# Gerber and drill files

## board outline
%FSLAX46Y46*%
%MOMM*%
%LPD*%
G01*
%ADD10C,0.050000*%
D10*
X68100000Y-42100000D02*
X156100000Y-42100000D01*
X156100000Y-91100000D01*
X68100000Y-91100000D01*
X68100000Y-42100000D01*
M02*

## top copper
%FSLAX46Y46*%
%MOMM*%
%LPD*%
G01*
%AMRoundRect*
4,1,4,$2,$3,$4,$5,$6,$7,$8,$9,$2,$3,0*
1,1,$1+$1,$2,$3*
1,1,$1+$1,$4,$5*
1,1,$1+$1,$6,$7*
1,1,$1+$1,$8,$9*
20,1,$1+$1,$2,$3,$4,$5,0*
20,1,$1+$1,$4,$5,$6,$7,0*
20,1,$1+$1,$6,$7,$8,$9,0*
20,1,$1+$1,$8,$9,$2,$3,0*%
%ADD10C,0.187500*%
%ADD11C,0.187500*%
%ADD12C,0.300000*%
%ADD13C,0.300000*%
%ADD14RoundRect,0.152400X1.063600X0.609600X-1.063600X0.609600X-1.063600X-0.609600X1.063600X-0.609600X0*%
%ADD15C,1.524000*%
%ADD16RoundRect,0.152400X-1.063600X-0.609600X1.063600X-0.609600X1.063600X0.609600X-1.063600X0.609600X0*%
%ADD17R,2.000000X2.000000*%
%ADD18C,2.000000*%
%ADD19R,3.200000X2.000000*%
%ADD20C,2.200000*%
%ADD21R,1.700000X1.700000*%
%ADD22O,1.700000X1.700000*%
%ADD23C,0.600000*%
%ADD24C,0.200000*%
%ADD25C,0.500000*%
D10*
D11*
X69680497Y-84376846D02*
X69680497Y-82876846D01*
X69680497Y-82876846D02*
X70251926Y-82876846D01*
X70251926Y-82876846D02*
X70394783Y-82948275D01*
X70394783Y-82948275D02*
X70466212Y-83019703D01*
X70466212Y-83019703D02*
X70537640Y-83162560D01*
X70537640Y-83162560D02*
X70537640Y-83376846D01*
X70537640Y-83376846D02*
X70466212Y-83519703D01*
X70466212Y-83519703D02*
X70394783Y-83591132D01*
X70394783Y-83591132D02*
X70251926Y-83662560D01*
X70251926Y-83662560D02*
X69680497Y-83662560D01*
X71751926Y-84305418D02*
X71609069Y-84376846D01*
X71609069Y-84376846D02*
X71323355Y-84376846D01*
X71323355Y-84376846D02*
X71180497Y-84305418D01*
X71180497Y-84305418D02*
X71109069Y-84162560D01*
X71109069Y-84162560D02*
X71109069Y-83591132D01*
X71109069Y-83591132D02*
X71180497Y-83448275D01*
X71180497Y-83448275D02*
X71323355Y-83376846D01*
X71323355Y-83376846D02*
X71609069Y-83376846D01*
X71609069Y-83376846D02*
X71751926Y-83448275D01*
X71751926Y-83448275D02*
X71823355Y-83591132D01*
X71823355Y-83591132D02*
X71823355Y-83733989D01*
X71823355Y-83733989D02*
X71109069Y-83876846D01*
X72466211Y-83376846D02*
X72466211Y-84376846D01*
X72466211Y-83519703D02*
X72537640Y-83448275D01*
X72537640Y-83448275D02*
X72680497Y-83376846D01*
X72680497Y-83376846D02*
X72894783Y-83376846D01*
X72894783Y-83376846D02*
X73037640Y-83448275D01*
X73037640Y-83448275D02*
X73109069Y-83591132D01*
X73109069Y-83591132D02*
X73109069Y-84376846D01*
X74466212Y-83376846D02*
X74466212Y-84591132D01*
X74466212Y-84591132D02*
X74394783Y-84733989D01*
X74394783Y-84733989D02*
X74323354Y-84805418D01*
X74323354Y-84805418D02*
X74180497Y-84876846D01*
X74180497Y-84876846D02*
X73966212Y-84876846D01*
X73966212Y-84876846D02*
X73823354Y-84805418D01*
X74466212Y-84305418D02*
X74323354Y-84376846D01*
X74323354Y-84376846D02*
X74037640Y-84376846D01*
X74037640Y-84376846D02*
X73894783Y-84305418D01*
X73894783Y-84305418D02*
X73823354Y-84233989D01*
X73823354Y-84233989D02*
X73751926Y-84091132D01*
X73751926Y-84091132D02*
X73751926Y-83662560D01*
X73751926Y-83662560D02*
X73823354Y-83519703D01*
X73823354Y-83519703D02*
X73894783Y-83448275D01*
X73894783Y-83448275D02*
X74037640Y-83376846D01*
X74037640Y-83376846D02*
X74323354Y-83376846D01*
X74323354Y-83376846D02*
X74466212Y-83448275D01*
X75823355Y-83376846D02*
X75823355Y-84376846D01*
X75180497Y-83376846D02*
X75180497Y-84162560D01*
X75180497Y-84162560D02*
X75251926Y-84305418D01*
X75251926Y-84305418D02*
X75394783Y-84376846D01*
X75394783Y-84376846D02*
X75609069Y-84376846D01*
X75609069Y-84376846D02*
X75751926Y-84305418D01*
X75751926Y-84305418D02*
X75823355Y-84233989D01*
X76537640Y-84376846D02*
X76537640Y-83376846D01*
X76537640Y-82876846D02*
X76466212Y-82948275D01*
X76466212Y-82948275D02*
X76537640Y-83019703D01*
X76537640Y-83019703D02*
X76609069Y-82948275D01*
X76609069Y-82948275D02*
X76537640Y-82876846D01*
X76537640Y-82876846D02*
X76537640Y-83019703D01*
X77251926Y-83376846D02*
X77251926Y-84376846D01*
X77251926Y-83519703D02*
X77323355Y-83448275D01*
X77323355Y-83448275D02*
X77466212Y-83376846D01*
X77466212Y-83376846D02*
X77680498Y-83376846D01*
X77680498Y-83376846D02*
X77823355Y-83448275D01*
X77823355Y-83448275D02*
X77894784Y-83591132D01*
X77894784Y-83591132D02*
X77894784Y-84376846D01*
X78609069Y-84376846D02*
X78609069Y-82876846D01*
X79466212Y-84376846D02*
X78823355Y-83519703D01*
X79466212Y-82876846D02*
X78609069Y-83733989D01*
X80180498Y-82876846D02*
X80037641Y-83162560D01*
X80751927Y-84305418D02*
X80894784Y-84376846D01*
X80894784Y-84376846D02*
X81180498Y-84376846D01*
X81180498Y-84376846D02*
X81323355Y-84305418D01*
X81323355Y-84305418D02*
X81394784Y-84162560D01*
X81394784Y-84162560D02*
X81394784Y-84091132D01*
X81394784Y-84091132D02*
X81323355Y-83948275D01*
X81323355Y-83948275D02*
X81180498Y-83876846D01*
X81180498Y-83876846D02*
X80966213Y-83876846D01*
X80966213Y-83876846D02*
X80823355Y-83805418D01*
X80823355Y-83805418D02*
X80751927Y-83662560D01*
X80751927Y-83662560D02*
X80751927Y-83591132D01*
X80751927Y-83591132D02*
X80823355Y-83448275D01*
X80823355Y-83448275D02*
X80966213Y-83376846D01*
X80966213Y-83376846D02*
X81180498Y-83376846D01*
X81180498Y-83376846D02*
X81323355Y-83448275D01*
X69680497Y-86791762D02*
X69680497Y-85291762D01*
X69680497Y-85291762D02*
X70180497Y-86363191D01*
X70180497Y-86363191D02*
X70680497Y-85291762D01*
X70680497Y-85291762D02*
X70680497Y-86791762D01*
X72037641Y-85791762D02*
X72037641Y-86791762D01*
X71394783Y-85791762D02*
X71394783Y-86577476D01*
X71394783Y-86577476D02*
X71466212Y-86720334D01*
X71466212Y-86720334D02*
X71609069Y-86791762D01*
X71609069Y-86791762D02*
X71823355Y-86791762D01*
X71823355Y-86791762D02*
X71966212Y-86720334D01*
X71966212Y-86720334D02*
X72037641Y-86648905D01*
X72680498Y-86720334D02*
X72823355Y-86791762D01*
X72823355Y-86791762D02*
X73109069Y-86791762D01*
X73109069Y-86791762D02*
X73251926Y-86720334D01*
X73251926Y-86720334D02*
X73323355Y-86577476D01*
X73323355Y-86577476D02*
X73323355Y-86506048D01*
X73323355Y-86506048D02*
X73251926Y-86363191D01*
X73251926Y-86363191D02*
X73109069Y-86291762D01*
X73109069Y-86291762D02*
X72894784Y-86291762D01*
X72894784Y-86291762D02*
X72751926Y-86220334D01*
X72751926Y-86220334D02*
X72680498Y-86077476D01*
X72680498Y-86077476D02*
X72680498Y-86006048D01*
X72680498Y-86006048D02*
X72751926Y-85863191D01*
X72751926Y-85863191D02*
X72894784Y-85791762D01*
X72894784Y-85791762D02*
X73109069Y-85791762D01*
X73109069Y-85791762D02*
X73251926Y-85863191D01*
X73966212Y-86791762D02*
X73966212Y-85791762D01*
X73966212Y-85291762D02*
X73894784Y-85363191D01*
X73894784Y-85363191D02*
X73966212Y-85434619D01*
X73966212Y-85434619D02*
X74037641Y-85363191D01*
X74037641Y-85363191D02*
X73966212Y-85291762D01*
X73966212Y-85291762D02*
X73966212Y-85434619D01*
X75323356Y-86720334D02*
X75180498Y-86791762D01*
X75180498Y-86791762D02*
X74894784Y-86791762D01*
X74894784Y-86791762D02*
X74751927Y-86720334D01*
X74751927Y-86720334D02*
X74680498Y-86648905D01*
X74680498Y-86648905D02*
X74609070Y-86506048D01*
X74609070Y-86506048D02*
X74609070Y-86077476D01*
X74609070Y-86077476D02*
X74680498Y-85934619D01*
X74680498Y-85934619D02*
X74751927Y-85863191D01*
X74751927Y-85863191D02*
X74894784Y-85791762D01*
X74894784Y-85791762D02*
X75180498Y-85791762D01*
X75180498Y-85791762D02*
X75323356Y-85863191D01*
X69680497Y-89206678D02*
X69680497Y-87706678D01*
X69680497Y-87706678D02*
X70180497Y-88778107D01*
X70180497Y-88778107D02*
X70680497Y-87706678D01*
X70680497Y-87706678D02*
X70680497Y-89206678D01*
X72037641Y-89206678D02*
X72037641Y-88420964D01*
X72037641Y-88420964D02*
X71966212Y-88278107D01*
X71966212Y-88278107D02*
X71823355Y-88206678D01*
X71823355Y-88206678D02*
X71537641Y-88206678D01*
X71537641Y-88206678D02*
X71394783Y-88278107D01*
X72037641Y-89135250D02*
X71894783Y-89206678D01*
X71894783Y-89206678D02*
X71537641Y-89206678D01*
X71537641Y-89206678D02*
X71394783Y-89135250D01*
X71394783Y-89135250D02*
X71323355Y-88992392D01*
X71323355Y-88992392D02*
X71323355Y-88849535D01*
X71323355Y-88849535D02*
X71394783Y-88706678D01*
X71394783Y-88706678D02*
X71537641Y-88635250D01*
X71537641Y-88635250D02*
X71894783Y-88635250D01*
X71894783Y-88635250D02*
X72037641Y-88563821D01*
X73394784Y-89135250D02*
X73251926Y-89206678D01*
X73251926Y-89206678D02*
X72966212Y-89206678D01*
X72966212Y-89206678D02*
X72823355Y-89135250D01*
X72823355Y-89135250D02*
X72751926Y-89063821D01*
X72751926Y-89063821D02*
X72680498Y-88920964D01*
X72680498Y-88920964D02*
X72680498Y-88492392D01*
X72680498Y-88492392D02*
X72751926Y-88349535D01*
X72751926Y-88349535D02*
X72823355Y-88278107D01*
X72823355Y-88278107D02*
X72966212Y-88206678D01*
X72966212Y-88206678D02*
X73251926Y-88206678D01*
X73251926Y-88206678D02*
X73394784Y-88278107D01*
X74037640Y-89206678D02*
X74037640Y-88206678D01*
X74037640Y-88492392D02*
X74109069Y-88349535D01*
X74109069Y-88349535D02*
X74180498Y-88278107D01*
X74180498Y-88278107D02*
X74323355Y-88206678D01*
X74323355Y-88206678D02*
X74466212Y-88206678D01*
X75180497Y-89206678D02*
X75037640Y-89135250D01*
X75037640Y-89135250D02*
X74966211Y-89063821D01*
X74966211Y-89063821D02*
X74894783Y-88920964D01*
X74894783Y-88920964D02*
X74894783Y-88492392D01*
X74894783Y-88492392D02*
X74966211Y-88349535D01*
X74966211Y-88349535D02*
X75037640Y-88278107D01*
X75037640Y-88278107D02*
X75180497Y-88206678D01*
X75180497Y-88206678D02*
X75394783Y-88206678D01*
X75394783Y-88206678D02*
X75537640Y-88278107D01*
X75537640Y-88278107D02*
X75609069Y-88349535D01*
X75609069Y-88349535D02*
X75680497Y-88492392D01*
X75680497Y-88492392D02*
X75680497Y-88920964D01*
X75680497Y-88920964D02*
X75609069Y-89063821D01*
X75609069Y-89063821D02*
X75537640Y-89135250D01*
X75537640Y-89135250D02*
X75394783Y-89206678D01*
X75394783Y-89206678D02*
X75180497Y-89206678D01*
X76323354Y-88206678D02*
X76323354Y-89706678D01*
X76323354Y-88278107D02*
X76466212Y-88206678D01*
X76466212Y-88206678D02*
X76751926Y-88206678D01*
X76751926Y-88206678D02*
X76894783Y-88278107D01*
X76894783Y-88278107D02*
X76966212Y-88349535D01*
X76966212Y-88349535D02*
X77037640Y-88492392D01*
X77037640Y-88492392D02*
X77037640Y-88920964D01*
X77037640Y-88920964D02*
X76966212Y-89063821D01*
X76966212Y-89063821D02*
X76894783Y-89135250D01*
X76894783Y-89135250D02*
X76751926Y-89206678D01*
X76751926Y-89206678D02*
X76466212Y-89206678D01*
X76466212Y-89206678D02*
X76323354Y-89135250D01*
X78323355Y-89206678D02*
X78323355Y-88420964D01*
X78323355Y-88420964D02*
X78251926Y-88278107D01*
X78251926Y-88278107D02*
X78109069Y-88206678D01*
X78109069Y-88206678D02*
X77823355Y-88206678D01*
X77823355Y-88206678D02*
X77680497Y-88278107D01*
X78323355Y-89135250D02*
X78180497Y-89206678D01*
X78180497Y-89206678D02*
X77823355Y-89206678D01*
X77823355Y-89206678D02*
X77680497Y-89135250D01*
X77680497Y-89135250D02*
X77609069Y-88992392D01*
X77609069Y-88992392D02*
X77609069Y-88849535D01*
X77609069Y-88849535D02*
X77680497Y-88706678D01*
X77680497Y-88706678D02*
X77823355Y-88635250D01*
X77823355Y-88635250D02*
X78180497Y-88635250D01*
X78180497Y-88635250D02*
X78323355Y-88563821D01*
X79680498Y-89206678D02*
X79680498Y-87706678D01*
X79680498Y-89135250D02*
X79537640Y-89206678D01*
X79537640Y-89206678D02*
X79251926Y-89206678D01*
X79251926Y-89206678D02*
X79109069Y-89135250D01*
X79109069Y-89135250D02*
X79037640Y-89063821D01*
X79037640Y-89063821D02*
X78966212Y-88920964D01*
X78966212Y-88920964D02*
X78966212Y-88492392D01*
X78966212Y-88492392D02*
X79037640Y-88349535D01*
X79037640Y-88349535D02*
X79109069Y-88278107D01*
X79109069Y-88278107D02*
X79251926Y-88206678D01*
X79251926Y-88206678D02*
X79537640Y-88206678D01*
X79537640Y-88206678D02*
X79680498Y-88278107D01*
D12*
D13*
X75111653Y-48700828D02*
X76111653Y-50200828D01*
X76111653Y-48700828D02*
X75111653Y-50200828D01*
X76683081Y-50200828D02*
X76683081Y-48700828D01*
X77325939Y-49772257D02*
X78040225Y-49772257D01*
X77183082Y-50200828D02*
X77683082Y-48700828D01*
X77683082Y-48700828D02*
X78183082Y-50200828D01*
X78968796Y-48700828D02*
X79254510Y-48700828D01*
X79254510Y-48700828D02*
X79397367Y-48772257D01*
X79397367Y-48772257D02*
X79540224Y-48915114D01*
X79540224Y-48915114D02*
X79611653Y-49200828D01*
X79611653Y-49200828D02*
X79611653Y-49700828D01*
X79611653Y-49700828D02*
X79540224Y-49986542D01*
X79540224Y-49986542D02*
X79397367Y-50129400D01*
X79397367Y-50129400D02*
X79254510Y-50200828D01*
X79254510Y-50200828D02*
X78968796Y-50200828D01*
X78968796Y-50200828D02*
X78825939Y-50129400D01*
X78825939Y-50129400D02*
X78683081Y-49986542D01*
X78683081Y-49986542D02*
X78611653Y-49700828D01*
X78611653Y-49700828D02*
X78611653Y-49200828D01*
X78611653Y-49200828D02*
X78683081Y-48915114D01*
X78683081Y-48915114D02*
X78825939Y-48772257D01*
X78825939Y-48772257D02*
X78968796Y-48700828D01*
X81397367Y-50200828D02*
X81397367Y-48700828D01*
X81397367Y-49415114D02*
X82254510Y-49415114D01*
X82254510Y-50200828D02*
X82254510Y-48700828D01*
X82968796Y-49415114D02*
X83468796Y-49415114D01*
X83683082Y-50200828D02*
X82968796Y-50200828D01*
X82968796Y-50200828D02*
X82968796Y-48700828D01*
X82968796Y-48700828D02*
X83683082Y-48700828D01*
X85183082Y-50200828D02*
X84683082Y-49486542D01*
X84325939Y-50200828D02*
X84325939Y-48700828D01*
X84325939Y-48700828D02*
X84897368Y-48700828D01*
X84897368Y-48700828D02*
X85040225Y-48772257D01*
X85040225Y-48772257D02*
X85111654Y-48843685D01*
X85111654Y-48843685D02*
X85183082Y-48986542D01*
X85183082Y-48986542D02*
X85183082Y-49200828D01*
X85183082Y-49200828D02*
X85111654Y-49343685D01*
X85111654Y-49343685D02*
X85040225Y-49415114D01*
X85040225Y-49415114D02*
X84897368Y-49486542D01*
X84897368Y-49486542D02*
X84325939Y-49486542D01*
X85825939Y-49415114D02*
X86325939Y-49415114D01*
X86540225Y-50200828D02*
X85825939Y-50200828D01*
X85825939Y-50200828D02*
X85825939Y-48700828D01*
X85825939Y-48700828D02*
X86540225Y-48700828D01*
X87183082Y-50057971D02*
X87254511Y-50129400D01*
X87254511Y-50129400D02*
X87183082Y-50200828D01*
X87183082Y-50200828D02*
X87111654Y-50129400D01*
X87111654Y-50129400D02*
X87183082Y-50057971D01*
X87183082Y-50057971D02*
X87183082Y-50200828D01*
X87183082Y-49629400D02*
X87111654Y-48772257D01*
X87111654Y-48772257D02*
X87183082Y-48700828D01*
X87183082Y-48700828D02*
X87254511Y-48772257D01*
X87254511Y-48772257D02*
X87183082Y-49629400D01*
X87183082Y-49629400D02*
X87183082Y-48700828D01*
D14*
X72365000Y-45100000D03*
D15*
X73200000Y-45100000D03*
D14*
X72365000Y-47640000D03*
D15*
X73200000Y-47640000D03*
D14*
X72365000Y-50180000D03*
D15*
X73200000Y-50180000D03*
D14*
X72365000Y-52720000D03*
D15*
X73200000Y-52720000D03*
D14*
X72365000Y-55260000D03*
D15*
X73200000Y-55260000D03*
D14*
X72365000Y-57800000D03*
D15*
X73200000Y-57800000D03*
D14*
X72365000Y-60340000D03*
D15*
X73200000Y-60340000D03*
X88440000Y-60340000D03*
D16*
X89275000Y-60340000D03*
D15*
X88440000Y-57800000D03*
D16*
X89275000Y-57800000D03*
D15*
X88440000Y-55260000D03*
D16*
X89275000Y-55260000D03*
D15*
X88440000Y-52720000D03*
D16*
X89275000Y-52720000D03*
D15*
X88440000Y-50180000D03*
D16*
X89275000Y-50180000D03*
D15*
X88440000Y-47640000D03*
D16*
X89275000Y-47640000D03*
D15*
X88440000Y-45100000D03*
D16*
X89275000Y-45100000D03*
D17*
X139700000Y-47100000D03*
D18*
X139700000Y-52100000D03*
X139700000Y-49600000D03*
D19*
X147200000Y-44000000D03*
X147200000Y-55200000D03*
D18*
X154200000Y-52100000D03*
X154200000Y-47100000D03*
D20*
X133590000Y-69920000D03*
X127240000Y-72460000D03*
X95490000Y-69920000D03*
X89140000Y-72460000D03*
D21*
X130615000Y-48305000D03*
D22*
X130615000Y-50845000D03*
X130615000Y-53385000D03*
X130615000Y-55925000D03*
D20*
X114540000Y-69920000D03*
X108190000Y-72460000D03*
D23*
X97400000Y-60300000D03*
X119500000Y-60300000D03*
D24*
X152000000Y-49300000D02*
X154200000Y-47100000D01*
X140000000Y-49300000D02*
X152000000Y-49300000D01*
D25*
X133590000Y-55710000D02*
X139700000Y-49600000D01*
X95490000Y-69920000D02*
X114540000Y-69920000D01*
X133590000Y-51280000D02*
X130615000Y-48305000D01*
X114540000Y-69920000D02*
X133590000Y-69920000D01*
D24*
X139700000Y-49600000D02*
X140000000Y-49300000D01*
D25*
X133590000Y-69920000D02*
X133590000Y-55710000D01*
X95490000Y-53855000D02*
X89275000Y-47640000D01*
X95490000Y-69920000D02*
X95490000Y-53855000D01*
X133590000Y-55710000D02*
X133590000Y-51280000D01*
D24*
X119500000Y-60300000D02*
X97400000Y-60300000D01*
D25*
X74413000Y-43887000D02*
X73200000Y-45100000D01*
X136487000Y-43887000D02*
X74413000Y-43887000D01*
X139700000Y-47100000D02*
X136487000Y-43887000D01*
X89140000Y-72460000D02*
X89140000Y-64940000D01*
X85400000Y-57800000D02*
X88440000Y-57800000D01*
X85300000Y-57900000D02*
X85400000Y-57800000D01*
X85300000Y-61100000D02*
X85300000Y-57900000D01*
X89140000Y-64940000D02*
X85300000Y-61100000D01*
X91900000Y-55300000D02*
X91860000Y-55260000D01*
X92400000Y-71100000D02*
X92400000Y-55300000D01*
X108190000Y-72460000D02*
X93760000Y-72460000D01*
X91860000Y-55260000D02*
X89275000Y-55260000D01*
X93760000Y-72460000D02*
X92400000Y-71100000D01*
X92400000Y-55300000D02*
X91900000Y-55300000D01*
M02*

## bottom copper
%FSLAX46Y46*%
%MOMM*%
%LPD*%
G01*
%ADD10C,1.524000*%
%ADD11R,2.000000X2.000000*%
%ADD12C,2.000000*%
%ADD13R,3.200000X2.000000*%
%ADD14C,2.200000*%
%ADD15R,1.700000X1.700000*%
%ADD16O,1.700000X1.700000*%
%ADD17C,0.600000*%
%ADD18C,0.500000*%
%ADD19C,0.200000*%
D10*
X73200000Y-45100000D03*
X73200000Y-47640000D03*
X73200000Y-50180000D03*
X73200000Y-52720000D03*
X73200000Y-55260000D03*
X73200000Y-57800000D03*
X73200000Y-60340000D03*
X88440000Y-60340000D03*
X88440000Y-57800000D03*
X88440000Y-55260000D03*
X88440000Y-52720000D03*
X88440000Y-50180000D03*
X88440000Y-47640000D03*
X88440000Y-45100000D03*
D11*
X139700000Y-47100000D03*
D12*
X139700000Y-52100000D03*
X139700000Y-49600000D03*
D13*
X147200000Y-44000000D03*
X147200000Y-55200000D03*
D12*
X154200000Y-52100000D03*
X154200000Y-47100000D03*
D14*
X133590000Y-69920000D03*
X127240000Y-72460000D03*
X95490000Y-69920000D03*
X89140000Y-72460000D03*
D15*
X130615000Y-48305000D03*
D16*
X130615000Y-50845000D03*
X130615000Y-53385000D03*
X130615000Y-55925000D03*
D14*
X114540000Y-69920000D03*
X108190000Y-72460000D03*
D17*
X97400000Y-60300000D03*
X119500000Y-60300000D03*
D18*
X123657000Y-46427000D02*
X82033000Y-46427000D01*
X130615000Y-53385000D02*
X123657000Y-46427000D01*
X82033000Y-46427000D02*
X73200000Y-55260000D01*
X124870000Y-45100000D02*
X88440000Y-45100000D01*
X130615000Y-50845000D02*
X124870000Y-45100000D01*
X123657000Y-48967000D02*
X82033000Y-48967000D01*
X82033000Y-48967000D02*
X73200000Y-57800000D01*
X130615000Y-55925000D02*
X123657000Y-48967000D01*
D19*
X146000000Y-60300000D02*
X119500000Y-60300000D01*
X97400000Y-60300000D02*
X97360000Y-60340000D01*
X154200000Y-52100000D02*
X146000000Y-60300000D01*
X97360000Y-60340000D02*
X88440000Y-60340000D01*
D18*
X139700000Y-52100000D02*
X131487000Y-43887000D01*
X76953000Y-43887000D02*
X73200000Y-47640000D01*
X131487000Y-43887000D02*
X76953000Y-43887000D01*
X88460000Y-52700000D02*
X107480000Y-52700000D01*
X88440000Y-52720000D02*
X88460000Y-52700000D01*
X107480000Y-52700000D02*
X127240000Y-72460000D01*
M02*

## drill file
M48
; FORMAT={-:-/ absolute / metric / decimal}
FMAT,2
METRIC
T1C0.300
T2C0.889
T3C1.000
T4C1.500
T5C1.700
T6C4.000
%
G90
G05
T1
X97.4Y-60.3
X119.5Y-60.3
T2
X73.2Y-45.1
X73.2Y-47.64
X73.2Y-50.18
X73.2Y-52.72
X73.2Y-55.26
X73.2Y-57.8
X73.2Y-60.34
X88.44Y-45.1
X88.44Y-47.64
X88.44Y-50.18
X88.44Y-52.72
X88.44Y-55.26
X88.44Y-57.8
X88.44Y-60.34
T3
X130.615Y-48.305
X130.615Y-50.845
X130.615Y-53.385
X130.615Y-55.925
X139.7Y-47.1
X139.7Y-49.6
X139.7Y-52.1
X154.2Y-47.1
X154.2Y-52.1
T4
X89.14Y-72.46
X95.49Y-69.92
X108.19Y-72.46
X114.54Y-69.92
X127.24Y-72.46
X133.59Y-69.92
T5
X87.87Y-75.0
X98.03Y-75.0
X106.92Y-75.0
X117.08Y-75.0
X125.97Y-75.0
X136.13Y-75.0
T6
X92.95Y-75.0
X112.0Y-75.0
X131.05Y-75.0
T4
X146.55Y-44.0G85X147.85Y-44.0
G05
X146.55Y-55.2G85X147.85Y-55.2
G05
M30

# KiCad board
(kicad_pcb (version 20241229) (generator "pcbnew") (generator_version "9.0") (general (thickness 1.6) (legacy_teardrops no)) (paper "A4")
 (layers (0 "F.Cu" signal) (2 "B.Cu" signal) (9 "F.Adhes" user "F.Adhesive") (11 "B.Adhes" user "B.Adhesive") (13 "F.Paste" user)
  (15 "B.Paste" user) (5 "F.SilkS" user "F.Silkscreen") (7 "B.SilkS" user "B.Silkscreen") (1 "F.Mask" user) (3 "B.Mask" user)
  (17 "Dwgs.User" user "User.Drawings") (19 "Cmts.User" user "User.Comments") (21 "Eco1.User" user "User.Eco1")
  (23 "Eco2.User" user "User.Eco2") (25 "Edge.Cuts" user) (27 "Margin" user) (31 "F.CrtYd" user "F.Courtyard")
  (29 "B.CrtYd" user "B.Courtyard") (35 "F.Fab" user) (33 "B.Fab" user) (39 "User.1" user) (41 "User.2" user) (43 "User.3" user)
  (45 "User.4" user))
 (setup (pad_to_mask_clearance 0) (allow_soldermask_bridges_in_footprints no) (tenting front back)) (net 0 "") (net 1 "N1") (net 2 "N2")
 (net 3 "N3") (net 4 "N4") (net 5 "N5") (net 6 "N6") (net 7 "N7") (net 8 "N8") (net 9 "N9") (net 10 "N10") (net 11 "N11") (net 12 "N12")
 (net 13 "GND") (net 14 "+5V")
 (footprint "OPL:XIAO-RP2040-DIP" (layer "F.Cu") (at 80.82 52.72)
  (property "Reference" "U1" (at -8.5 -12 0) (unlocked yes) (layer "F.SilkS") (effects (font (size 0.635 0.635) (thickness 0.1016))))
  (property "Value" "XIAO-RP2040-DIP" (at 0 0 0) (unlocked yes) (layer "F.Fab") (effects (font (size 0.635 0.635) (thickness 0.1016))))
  (pad "1" smd roundrect (at -8.455 -7.62 180) (size 2.432 1.524) (layers "F.Cu" "F.Mask") (roundrect_rratio 0.1) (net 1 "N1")
   (thermal_bridge_angle 45))
  (pad "1" thru_hole circle (at -7.62 -7.62 180) (size 1.524 1.524) (drill 0.889) (layers "*.Cu" "*.Mask") (remove_unused_layers no)
   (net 1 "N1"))
  (pad "2" smd roundrect (at -8.455 -5.08 180) (size 2.432 1.524) (layers "F.Cu" "F.Mask") (roundrect_rratio 0.1) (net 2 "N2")
   (thermal_bridge_angle 45))
  (pad "2" thru_hole circle (at -7.62 -5.08 180) (size 1.524 1.524) (drill 0.889) (layers "*.Cu" "*.Mask") (remove_unused_layers no)
   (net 2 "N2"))
  (pad "3" smd roundrect (at -8.455 -2.54 180) (size 2.432 1.524) (layers "F.Cu" "F.Mask") (roundrect_rratio 0.1) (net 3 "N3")
   (thermal_bridge_angle 45))
  (pad "3" thru_hole circle (at -7.62 -2.54 180) (size 1.524 1.524) (drill 0.889) (layers "*.Cu" "*.Mask") (remove_unused_layers no)
   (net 3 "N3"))
  (pad "4" smd roundrect (at -8.455 0 180) (size 2.432 1.524) (layers "F.Cu" "F.Mask") (roundrect_rratio 0.1) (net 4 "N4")
   (thermal_bridge_angle 45))
  (pad "4" thru_hole circle (at -7.62 0 180) (size 1.524 1.524) (drill 0.889) (layers "*.Cu" "*.Mask") (remove_unused_layers no)
   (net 4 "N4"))
  (pad "5" smd roundrect (at -8.455 2.54 180) (size 2.432 1.524) (layers "F.Cu" "F.Mask") (roundrect_rratio 0.1) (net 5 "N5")
   (thermal_bridge_angle 45))
  (pad "5" thru_hole circle (at -7.62 2.54 180) (size 1.524 1.524) (drill 0.889) (layers "*.Cu" "*.Mask") (remove_unused_layers no)
   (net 5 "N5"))
  (pad "6" smd roundrect (at -8.455 5.08 180) (size 2.432 1.524) (layers "F.Cu" "F.Mask") (roundrect_rratio 0.1) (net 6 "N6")
   (thermal_bridge_angle 45))
  (pad "6" thru_hole circle (at -7.62 5.08 180) (size 1.524 1.524) (drill 0.889) (layers "*.Cu" "*.Mask") (remove_unused_layers no)
   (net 6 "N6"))
  (pad "7" smd roundrect (at -8.455 7.62 180) (size 2.432 1.524) (layers "F.Cu" "F.Mask") (roundrect_rratio 0.1) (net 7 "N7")
   (thermal_bridge_angle 45))
  (pad "7" thru_hole circle (at -7.62 7.62 180) (size 1.524 1.524) (drill 0.889) (layers "*.Cu" "*.Mask") (remove_unused_layers no)
   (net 7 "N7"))
  (pad "8" thru_hole circle (at 7.62 7.62) (size 1.524 1.524) (drill 0.889) (layers "*.Cu" "*.Mask") (remove_unused_layers no) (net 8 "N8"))
  (pad "8" smd roundrect (at 8.455 7.62) (size 2.432 1.524) (layers "F.Cu" "F.Mask") (roundrect_rratio 0.1) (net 8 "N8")
   (thermal_bridge_angle 45))
  (pad "9" thru_hole circle (at 7.62 5.08) (size 1.524 1.524) (drill 0.889) (layers "*.Cu" "*.Mask") (remove_unused_layers no) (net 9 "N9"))
  (pad "9" smd roundrect (at 8.455 5.08) (size 2.432 1.524) (layers "F.Cu" "F.Mask") (roundrect_rratio 0.1) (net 9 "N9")
   (thermal_bridge_angle 45))
  (pad "10" thru_hole circle (at 7.62 2.54) (size 1.524 1.524) (drill 0.889) (layers "*.Cu" "*.Mask") (remove_unused_layers no)
   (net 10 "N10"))
  (pad "10" smd roundrect (at 8.455 2.54) (size 2.432 1.524) (layers "F.Cu" "F.Mask") (roundrect_rratio 0.1) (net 10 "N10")
   (thermal_bridge_angle 45))
  (pad "11" thru_hole circle (at 7.62 0) (size 1.524 1.524) (drill 0.889) (layers "*.Cu" "*.Mask") (remove_unused_layers no) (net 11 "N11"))
  (pad "11" smd roundrect (at 8.455 0) (size 2.432 1.524) (layers "F.Cu" "F.Mask") (roundrect_rratio 0.1) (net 11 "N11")
   (thermal_bridge_angle 45))
  (pad "12" thru_hole circle (at 7.62 -2.54) (size 1.524 1.524) (drill 0.889) (layers "*.Cu" "*.Mask") (remove_unused_layers no)
   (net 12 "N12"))
  (pad "12" smd roundrect (at 8.455 -2.54) (size 2.432 1.524) (layers "F.Cu" "F.Mask") (roundrect_rratio 0.1) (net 12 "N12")
   (thermal_bridge_angle 45))
  (pad "13" thru_hole circle (at 7.62 -5.08) (size 1.524 1.524) (drill 0.889) (layers "*.Cu" "*.Mask") (remove_unused_layers no)
   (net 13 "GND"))
  (pad "13" smd roundrect (at 8.455 -5.08) (size 2.432 1.524) (layers "F.Cu" "F.Mask") (roundrect_rratio 0.1) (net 13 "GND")
   (thermal_bridge_angle 45))
  (pad "14" thru_hole circle (at 7.62 -7.62) (size 1.524 1.524) (drill 0.889) (layers "*.Cu" "*.Mask") (remove_unused_layers no)
   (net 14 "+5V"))
  (pad "14" smd roundrect (at 8.455 -7.62) (size 2.432 1.524) (layers "F.Cu" "F.Mask") (roundrect_rratio 0.1) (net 14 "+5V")
   (thermal_bridge_angle 45)))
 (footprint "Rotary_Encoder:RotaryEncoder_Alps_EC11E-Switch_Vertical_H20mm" (layer "F.Cu") (at 139.7 47.1)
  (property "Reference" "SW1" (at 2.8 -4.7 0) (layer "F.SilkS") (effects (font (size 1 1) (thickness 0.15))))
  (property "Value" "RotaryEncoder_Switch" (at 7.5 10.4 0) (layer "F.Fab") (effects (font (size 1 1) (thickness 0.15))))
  (pad "A" thru_hole rect (at 0 0) (size 2 2) (drill 1) (layers "*.Cu" "*.Mask") (remove_unused_layers no) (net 1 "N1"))
  (pad "B" thru_hole circle (at 0 5) (size 2 2) (drill 1) (layers "*.Cu" "*.Mask") (remove_unused_layers no) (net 2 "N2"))
  (pad "C" thru_hole circle (at 0 2.5) (size 2 2) (drill 1) (layers "*.Cu" "*.Mask") (remove_unused_layers no) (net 13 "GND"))
  (pad "MP" thru_hole rect (at 7.5 -3.1) (size 3.2 2) (drill oval 2.8 1.5) (layers "*.Cu" "*.Mask") (remove_unused_layers no))
  (pad "MP" thru_hole rect (at 7.5 8.1) (size 3.2 2) (drill oval 2.8 1.5) (layers "*.Cu" "*.Mask") (remove_unused_layers no))
  (pad "S1" thru_hole circle (at 14.5 5) (size 2 2) (drill 1) (layers "*.Cu" "*.Mask") (remove_unused_layers no) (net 8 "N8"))
  (pad "S2" thru_hole circle (at 14.5 0) (size 2 2) (drill 1) (layers "*.Cu" "*.Mask") (remove_unused_layers no) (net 13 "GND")))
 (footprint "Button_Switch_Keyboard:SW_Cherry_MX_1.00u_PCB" (layer "F.Cu") (at 133.59 69.92)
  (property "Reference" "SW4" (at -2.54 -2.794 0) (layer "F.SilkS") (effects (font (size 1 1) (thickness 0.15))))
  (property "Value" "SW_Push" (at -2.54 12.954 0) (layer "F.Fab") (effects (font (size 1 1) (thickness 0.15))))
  (pad "" np_thru_hole circle (at -7.62 5.08) (size 1.7 1.7) (drill 1.7) (layers "*.Cu" "*.Mask"))
  (pad "" np_thru_hole circle (at -2.54 5.08) (size 4 4) (drill 4) (layers "*.Cu" "*.Mask"))
  (pad "" np_thru_hole circle (at 2.54 5.08) (size 1.7 1.7) (drill 1.7) (layers "*.Cu" "*.Mask"))
  (pad "1" thru_hole circle (at 0 0) (size 2.2 2.2) (drill 1.5) (layers "*.Cu" "*.Mask") (remove_unused_layers no) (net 13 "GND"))
  (pad "2" thru_hole circle (at -6.35 2.54) (size 2.2 2.2) (drill 1.5) (layers "*.Cu" "*.Mask") (remove_unused_layers no) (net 11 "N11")))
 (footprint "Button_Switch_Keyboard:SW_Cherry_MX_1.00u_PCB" (layer "F.Cu") (at 95.49 69.92)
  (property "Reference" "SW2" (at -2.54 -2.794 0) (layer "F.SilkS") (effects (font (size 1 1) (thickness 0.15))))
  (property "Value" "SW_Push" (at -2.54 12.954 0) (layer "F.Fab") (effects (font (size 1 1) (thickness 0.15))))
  (pad "" np_thru_hole circle (at -7.62 5.08) (size 1.7 1.7) (drill 1.7) (layers "*.Cu" "*.Mask"))
  (pad "" np_thru_hole circle (at -2.54 5.08) (size 4 4) (drill 4) (layers "*.Cu" "*.Mask"))
  (pad "" np_thru_hole circle (at 2.54 5.08) (size 1.7 1.7) (drill 1.7) (layers "*.Cu" "*.Mask"))
  (pad "1" thru_hole circle (at 0 0) (size 2.2 2.2) (drill 1.5) (layers "*.Cu" "*.Mask") (remove_unused_layers no) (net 13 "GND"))
  (pad "2" thru_hole circle (at -6.35 2.54) (size 2.2 2.2) (drill 1.5) (layers "*.Cu" "*.Mask") (remove_unused_layers no) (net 9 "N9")))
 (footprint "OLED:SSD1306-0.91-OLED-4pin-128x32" (layer "F.Cu") (at 94.115 46.115)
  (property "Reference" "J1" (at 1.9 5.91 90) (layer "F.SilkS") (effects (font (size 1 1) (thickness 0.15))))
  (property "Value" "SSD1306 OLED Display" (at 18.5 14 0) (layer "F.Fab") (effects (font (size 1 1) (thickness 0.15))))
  (pad "1" thru_hole rect (at 36.5 2.19) (size 1.7 1.7) (drill 1) (layers "*.Cu" "*.Mask") (remove_unused_layers no) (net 13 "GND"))
  (pad "2" thru_hole oval (at 36.5 4.73) (size 1.7 1.7) (drill 1) (layers "*.Cu" "*.Mask") (remove_unused_layers no) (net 14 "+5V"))
  (pad "3" thru_hole oval (at 36.5 7.27) (size 1.7 1.7) (drill 1) (layers "*.Cu" "*.Mask") (remove_unused_layers no) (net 5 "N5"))
  (pad "4" thru_hole oval (at 36.5 9.81) (size 1.7 1.7) (drill 1) (layers "*.Cu" "*.Mask") (remove_unused_layers no) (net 6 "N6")))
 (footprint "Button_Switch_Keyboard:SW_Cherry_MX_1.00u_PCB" (layer "F.Cu") (at 114.54 69.92)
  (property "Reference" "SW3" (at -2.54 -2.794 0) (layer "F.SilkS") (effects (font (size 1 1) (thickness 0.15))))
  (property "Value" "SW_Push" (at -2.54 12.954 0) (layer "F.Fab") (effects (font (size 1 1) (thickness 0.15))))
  (pad "" np_thru_hole circle (at -7.62 5.08) (size 1.7 1.7) (drill 1.7) (layers "*.Cu" "*.Mask"))
  (pad "" np_thru_hole circle (at -2.54 5.08) (size 4 4) (drill 4) (layers "*.Cu" "*.Mask"))
  (pad "" np_thru_hole circle (at 2.54 5.08) (size 1.7 1.7) (drill 1.7) (layers "*.Cu" "*.Mask"))
  (pad "1" thru_hole circle (at 0 0) (size 2.2 2.2) (drill 1.5) (layers "*.Cu" "*.Mask") (remove_unused_layers no) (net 13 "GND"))
  (pad "2" thru_hole circle (at -6.35 2.54) (size 2.2 2.2) (drill 1.5) (layers "*.Cu" "*.Mask") (remove_unused_layers no) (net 10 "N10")))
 (gr_rect (start 68.1 42.1) (end 156.1 91.1) (stroke (width 0.05) (type solid)) (fill no) (layer "Edge.Cuts"))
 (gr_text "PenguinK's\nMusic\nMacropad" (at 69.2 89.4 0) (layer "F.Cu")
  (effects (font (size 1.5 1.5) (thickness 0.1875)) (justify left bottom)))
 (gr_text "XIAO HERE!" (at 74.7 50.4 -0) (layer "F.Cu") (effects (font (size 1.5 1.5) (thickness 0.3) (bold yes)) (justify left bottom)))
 (segment (start 123.657 46.427) (end 82.033 46.427) (width 0.5) (layer "B.Cu") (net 5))
 (segment (start 130.615 53.385) (end 123.657 46.427) (width 0.5) (layer "B.Cu") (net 5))
 (segment (start 82.033 46.427) (end 73.2 55.26) (width 0.5) (layer "B.Cu") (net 5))
 (segment (start 124.87 45.1) (end 88.44 45.1) (width 0.5) (layer "B.Cu") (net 14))
 (segment (start 130.615 50.845) (end 124.87 45.1) (width 0.5) (layer "B.Cu") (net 14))
 (segment (start 152 49.3) (end 154.2 47.1) (width 0.2) (layer "F.Cu") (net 13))
 (segment (start 140 49.3) (end 152 49.3) (width 0.2) (layer "F.Cu") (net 13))
 (segment (start 133.59 55.71) (end 139.7 49.6) (width 0.5) (layer "F.Cu") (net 13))
 (segment (start 95.49 69.92) (end 114.54 69.92) (width 0.5) (layer "F.Cu") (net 13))
 (segment (start 133.59 51.28) (end 130.615 48.305) (width 0.5) (layer "F.Cu") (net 13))
 (segment (start 114.54 69.92) (end 133.59 69.92) (width 0.5) (layer "F.Cu") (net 13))
 (segment (start 139.7 49.6) (end 140 49.3) (width 0.2) (layer "F.Cu") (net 13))
 (segment (start 133.59 69.92) (end 133.59 55.71) (width 0.5) (layer "F.Cu") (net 13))
 (segment (start 95.49 53.855) (end 89.275 47.64) (width 0.5) (layer "F.Cu") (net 13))
 (segment (start 95.49 69.92) (end 95.49 53.855) (width 0.5) (layer "F.Cu") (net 13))
 (segment (start 133.59 55.71) (end 133.59 51.28) (width 0.5) (layer "F.Cu") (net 13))
 (segment (start 123.657 48.967) (end 82.033 48.967) (width 0.5) (layer "B.Cu") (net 6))
 (segment (start 82.033 48.967) (end 73.2 57.8) (width 0.5) (layer "B.Cu") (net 6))
 (segment (start 130.615 55.925) (end 123.657 48.967) (width 0.5) (layer "B.Cu") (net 6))
 (segment (start 119.5 60.3) (end 97.4 60.3) (width 0.2) (layer "F.Cu") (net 8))
 (via (at 97.4 60.3) (size 0.6) (drill 0.3) (layers "F.Cu" "B.Cu") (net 8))
 (via (at 119.5 60.3) (size 0.6) (drill 0.3) (layers "F.Cu" "B.Cu") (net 8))
 (segment (start 146 60.3) (end 119.5 60.3) (width 0.2) (layer "B.Cu") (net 8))
 (segment (start 97.4 60.3) (end 97.36 60.34) (width 0.2) (layer "B.Cu") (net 8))
 (segment (start 154.2 52.1) (end 146 60.3) (width 0.2) (layer "B.Cu") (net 8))
 (segment (start 97.36 60.34) (end 88.44 60.34) (width 0.2) (layer "B.Cu") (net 8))
 (segment (start 74.413 43.887) (end 73.2 45.1) (width 0.5) (layer "F.Cu") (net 1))
 (segment (start 136.487 43.887) (end 74.413 43.887) (width 0.5) (layer "F.Cu") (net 1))
 (segment (start 139.7 47.1) (end 136.487 43.887) (width 0.5) (layer "F.Cu") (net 1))
 (segment (start 139.7 52.1) (end 131.487 43.887) (width 0.5) (layer "B.Cu") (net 2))
 (segment (start 76.953 43.887) (end 73.2 47.64) (width 0.5) (layer "B.Cu") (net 2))
 (segment (start 131.487 43.887) (end 76.953 43.887) (width 0.5) (layer "B.Cu") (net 2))
 (segment (start 89.14 72.46) (end 89.14 64.94) (width 0.5) (layer "F.Cu") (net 9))
 (segment (start 85.4 57.8) (end 88.44 57.8) (width 0.5) (layer "F.Cu") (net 9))
 (segment (start 85.3 57.9) (end 85.4 57.8) (width 0.5) (layer "F.Cu") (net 9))
 (segment (start 85.3 61.1) (end 85.3 57.9) (width 0.5) (layer "F.Cu") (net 9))
 (segment (start 89.14 64.94) (end 85.3 61.1) (width 0.5) (layer "F.Cu") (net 9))
 (segment (start 91.9 55.3) (end 91.86 55.26) (width 0.5) (layer "F.Cu") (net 10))
 (segment (start 92.4 71.1) (end 92.4 55.3) (width 0.5) (layer "F.Cu") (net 10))
 (segment (start 108.19 72.46) (end 93.76 72.46) (width 0.5) (layer "F.Cu") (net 10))
 (segment (start 91.86 55.26) (end 89.275 55.26) (width 0.5) (layer "F.Cu") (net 10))
 (segment (start 93.76 72.46) (end 92.4 71.1) (width 0.5) (layer "F.Cu") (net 10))
 (segment (start 92.4 55.3) (end 91.9 55.3) (width 0.5) (layer "F.Cu") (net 10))
 (segment (start 88.46 52.7) (end 107.48 52.7) (width 0.5) (layer "B.Cu") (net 11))
 (segment (start 88.44 52.72) (end 88.46 52.7) (width 0.5) (layer "B.Cu") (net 11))
 (segment (start 107.48 52.7) (end 127.24 72.46) (width 0.5) (layer "B.Cu") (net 11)))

